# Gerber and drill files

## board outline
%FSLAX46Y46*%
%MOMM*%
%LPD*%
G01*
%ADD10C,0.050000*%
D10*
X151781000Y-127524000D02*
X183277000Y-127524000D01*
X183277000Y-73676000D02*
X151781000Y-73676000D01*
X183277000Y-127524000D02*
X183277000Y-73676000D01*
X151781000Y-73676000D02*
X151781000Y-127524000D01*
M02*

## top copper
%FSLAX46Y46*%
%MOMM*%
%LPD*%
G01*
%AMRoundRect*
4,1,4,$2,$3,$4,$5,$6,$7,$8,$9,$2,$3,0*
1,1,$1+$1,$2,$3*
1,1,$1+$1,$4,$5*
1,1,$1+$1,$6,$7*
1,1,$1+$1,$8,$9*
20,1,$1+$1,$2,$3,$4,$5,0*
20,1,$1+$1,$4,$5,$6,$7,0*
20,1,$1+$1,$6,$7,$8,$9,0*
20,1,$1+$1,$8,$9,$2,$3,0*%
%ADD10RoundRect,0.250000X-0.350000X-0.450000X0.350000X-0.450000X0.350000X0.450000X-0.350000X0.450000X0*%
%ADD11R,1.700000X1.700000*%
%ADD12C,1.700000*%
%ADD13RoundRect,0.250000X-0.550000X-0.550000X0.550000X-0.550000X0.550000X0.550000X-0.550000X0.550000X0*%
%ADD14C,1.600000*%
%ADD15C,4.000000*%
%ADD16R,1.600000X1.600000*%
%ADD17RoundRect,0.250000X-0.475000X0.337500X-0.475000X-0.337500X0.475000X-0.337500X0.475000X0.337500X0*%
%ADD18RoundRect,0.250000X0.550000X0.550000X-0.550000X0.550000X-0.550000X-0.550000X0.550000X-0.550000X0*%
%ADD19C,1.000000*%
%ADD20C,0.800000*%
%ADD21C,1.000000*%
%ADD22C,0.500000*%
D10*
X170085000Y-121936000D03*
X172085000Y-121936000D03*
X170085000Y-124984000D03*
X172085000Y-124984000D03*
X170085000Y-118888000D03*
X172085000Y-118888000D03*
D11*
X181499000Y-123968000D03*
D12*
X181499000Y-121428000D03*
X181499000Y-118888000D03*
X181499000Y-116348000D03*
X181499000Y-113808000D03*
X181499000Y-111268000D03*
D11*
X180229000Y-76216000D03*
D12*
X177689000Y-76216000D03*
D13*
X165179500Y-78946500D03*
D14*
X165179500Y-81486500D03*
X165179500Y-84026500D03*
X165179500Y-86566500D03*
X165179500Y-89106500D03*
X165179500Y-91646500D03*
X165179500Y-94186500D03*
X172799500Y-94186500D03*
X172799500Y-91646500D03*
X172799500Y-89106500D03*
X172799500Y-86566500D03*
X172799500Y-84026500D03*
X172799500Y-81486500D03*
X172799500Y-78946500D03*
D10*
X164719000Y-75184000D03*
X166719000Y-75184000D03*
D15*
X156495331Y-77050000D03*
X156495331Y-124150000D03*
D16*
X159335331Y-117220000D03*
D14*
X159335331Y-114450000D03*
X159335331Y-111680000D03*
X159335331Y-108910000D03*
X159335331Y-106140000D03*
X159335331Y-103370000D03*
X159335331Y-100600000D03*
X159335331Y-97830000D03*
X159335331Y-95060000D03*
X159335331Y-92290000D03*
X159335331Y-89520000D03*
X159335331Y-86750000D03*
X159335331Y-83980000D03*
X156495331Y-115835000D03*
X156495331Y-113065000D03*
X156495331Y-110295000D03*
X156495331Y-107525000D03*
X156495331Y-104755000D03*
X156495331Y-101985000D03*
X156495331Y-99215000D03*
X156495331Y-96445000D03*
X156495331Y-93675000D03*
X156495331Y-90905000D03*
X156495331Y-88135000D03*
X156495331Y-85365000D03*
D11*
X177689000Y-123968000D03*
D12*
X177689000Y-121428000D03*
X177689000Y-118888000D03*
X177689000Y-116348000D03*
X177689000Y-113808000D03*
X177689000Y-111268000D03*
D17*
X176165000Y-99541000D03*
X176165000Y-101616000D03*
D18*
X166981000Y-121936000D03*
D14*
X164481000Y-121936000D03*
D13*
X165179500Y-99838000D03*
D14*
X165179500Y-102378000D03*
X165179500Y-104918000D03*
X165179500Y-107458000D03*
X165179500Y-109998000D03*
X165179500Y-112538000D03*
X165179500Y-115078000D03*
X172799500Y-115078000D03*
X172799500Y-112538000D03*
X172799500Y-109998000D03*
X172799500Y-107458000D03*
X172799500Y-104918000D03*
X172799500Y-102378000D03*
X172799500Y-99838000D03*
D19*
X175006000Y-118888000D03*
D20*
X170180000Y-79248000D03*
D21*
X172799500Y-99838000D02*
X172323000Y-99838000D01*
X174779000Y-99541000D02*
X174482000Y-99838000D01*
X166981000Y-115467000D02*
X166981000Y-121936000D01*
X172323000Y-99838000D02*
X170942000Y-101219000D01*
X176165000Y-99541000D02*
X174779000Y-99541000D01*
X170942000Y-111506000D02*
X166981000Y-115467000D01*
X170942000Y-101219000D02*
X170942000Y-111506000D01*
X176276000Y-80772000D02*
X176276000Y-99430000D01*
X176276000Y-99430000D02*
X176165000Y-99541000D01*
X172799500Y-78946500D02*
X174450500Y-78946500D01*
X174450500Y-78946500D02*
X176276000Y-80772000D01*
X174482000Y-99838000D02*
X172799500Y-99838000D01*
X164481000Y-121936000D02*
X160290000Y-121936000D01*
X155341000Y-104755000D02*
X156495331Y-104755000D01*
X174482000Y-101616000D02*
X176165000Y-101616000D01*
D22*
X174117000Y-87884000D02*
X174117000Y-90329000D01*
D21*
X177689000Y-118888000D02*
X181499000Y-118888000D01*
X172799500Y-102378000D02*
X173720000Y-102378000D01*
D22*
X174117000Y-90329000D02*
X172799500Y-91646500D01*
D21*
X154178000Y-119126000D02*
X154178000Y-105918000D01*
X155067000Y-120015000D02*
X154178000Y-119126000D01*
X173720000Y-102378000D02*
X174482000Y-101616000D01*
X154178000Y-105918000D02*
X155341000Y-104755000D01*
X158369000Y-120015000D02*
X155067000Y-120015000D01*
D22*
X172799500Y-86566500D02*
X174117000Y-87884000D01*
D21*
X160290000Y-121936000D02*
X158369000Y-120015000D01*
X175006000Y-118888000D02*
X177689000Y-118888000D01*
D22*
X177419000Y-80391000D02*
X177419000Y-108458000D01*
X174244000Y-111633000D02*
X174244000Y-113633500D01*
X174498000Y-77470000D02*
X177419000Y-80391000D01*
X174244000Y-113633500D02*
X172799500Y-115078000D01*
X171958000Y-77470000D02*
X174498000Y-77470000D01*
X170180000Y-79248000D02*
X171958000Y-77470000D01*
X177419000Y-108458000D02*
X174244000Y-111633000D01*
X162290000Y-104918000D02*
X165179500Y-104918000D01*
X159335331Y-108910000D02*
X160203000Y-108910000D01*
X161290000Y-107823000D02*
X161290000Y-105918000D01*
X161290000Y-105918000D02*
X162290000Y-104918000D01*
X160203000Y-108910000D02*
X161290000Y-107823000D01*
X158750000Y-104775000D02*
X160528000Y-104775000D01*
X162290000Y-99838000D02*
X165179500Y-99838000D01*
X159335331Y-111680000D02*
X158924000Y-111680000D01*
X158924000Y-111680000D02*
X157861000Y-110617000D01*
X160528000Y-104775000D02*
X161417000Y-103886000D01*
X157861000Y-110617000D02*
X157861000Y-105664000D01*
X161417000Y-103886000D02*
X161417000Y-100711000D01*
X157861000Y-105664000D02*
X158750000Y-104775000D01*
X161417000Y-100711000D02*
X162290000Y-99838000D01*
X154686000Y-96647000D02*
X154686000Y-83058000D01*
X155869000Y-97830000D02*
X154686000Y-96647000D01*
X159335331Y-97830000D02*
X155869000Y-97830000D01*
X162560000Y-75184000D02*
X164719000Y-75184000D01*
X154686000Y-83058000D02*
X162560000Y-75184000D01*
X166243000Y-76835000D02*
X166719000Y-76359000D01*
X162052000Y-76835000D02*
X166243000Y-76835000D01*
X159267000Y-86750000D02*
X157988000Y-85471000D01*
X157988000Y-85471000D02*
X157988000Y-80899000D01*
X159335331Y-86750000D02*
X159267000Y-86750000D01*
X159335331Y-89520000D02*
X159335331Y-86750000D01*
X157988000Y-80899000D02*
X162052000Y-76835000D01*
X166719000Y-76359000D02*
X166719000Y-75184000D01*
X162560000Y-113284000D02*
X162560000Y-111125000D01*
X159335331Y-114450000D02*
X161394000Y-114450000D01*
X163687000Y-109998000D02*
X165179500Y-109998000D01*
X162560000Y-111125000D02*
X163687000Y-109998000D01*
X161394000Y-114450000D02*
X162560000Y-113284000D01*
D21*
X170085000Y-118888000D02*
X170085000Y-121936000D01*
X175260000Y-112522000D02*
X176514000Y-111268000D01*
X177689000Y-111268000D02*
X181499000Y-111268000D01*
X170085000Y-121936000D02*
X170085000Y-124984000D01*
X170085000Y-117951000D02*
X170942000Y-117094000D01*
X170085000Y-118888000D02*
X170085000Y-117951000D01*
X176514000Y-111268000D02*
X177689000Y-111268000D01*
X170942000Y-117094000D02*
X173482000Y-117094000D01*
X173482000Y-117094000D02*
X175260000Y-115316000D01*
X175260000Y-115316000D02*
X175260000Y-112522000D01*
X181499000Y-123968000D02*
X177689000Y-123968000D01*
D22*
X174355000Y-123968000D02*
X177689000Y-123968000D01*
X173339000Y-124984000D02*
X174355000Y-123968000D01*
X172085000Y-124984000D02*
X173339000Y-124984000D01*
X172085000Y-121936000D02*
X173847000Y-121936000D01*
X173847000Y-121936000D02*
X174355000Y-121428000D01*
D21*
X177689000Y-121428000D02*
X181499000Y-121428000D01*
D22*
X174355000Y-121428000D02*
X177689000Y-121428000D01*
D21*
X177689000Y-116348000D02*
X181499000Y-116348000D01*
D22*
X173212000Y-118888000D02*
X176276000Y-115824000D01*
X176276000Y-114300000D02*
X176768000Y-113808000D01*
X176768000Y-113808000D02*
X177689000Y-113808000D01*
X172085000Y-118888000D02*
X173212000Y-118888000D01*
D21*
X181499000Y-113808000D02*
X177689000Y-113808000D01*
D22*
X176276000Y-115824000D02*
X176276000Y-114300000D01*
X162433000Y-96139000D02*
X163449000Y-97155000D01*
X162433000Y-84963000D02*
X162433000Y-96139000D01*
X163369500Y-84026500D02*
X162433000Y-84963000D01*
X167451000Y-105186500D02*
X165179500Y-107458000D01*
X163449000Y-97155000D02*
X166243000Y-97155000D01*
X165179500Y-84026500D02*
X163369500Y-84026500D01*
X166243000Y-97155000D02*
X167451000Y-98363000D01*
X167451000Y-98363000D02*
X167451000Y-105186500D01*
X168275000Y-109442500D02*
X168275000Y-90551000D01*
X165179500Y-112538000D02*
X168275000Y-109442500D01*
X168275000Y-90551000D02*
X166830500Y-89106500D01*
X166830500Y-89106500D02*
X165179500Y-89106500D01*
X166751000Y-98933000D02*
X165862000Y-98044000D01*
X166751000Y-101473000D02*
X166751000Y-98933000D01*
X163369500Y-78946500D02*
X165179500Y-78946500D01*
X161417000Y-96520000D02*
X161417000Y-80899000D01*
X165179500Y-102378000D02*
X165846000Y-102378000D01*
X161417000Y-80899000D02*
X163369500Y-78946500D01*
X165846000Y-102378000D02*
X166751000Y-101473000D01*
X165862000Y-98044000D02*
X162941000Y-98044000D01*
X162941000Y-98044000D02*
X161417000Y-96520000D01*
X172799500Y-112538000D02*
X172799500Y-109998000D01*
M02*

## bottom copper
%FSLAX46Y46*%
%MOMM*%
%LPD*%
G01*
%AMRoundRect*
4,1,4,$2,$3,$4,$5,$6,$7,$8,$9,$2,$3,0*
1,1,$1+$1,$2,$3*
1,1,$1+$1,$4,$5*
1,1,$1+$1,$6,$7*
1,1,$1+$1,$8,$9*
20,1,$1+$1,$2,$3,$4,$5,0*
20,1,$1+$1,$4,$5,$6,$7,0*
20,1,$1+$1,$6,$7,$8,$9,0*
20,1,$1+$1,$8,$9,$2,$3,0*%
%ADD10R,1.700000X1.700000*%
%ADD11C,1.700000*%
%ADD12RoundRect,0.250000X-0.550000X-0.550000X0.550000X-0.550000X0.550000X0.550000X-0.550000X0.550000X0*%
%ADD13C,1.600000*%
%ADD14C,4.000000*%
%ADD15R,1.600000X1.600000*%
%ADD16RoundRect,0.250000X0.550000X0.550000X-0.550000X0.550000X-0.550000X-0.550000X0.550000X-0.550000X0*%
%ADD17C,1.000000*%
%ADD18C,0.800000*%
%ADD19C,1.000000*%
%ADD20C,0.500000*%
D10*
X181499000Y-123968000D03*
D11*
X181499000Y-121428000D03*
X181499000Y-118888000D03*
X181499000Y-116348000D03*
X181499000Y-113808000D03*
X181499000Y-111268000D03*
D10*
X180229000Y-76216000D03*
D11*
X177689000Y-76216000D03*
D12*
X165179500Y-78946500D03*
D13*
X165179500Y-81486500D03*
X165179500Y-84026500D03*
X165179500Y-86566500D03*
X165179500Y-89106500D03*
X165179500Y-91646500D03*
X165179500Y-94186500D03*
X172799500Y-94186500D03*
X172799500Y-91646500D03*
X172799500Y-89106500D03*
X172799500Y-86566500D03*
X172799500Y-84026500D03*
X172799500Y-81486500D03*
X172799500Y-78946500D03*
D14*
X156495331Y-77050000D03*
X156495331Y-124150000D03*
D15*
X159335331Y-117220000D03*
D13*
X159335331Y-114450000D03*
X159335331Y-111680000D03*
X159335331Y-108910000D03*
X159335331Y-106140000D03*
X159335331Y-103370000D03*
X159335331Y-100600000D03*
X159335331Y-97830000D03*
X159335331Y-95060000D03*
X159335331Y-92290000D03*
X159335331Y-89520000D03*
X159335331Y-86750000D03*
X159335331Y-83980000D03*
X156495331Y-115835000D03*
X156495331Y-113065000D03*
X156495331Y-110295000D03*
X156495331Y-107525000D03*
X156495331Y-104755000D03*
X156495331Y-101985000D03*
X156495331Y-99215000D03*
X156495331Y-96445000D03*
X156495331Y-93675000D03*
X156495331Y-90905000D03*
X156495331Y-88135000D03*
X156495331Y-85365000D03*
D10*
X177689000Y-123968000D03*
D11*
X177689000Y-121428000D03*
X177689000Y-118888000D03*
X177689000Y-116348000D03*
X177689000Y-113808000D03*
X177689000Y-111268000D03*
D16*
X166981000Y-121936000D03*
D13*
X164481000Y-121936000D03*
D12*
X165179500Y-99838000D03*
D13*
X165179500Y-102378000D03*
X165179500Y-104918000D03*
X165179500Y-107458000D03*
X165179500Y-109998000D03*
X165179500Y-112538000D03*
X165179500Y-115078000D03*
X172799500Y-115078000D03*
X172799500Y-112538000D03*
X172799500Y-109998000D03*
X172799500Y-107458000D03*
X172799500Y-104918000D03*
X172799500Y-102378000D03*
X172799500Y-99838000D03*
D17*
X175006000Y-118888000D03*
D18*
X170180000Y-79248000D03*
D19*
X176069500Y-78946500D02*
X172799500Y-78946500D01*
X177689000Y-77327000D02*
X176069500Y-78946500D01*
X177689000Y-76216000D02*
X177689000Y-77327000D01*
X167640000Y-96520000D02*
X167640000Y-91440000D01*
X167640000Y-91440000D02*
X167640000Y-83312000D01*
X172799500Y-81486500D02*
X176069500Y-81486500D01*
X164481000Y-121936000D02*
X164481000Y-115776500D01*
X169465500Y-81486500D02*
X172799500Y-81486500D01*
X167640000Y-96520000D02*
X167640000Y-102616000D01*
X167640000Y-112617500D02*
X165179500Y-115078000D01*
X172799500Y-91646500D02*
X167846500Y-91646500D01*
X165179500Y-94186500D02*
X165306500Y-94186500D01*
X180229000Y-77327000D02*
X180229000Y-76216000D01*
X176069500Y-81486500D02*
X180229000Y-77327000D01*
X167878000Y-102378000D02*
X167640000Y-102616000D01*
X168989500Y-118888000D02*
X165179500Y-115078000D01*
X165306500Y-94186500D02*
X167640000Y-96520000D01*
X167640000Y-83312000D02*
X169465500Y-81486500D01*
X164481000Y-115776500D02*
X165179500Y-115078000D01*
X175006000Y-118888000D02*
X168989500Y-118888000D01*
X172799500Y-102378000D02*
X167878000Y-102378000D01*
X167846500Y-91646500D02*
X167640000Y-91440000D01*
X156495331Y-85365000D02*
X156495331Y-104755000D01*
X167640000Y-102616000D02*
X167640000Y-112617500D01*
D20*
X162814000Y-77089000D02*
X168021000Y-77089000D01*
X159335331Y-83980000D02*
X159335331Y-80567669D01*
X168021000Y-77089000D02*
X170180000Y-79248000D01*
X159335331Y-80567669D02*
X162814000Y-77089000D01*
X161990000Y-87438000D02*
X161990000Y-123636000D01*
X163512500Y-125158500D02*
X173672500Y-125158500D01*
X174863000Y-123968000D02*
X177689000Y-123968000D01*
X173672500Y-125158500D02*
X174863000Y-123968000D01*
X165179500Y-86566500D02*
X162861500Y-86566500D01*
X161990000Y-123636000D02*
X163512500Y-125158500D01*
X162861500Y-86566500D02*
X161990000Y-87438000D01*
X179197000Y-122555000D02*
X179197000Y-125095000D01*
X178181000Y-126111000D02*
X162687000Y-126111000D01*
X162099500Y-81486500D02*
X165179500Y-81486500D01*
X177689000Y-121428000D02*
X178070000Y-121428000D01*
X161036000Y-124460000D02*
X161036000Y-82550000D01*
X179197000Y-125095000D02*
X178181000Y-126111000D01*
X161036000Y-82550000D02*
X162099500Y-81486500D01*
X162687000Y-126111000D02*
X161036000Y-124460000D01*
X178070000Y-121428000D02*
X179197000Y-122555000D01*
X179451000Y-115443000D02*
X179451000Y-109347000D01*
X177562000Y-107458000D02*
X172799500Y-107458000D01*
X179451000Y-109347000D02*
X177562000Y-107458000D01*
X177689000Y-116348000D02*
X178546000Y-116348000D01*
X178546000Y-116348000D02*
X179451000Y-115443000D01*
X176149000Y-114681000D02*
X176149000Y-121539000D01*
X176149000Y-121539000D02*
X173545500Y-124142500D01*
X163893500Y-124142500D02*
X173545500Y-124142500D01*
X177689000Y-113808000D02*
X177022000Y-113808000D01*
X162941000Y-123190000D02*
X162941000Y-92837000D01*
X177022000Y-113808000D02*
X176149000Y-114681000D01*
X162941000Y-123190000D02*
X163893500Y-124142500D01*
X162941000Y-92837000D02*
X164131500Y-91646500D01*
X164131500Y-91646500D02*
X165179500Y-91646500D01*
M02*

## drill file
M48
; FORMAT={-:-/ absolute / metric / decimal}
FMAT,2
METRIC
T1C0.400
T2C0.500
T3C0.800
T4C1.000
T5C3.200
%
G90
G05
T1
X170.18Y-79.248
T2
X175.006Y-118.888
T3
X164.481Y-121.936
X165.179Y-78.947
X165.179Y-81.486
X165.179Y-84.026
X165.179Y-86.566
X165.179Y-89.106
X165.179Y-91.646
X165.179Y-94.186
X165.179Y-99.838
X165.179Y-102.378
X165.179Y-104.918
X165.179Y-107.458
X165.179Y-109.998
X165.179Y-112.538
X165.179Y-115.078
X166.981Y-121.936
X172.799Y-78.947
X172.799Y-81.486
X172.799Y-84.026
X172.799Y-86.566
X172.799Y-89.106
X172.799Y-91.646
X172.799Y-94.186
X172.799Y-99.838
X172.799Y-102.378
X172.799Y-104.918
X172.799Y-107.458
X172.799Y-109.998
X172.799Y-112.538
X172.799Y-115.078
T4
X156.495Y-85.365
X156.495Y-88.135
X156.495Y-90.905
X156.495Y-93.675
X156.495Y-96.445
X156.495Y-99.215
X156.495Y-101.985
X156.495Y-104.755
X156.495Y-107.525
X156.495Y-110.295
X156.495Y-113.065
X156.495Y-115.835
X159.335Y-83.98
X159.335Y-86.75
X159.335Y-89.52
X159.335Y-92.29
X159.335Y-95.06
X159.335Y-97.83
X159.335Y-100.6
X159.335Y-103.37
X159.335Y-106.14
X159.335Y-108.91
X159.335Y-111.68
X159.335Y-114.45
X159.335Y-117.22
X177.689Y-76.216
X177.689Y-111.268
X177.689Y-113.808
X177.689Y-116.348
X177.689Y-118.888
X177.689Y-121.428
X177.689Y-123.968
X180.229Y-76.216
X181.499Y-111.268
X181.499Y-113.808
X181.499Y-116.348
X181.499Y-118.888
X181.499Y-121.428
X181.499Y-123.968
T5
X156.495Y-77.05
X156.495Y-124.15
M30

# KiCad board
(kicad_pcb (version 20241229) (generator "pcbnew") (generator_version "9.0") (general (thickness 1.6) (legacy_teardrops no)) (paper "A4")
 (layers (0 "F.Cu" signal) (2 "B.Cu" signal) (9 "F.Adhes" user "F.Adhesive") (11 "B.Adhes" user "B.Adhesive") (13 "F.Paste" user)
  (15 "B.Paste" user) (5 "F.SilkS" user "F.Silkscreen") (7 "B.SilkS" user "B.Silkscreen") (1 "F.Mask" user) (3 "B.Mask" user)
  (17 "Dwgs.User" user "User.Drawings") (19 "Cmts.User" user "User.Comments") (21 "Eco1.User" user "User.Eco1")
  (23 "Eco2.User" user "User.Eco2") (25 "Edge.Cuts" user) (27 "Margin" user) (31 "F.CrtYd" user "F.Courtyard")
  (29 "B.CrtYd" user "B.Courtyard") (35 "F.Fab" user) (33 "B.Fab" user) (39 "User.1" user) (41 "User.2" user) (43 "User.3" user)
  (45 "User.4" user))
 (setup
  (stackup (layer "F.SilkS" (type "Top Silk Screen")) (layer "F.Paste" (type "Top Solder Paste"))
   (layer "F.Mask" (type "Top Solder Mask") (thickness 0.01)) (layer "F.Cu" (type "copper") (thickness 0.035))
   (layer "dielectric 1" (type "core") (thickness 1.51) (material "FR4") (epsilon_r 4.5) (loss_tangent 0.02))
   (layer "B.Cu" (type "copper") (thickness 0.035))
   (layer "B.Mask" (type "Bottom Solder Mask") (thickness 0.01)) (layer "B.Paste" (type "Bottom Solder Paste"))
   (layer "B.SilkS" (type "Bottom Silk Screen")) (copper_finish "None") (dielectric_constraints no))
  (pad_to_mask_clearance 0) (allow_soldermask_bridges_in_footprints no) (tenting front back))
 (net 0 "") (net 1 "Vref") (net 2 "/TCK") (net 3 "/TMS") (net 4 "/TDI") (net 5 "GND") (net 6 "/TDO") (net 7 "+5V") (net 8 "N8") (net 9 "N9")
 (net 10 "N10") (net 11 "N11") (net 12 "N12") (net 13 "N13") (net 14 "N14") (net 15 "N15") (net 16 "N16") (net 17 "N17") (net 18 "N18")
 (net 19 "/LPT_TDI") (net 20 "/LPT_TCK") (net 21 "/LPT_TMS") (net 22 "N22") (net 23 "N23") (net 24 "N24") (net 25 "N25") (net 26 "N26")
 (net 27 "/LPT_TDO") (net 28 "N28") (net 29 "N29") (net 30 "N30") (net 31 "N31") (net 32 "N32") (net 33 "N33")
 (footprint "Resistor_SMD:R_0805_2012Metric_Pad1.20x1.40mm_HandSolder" (layer "F.Cu") (at 171.085 121.936)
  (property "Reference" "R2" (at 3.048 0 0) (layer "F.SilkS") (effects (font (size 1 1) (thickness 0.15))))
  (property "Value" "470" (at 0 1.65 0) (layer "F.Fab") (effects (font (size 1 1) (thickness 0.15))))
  (pad "1" smd roundrect (at -1 0) (size 1.2 1.4) (layers "F.Cu" "F.Mask" "F.Paste") (roundrect_rratio 0.208333) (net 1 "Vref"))
  (pad "2" smd roundrect (at 1 0) (size 1.2 1.4) (layers "F.Cu" "F.Mask" "F.Paste") (roundrect_rratio 0.208333) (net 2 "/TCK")))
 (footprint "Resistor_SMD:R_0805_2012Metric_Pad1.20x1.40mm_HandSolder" (layer "F.Cu") (at 171.085 124.984)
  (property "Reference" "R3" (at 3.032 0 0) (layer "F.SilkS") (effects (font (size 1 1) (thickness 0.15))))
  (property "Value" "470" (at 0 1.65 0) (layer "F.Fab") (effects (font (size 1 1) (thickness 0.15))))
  (pad "1" smd roundrect (at -1 0) (size 1.2 1.4) (layers "F.Cu" "F.Mask" "F.Paste") (roundrect_rratio 0.208333) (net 1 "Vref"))
  (pad "2" smd roundrect (at 1 0) (size 1.2 1.4) (layers "F.Cu" "F.Mask" "F.Paste") (roundrect_rratio 0.208333) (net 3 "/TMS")))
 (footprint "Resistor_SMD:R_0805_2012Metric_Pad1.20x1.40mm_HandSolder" (layer "F.Cu") (at 171.085 118.888)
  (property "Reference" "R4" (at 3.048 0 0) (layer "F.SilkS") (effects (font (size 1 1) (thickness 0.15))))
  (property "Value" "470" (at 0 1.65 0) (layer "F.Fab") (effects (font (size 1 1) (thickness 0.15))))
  (pad "1" smd roundrect (at -1 0) (size 1.2 1.4) (layers "F.Cu" "F.Mask" "F.Paste") (roundrect_rratio 0.208333) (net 1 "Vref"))
  (pad "2" smd roundrect (at 1 0) (size 1.2 1.4) (layers "F.Cu" "F.Mask" "F.Paste") (roundrect_rratio 0.208333) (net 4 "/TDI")))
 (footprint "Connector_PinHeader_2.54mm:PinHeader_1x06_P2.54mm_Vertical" (layer "F.Cu") (at 181.499 123.968 180)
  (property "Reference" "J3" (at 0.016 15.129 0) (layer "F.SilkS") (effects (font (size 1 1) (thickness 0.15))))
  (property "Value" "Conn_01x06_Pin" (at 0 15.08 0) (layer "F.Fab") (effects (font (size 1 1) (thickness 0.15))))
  (pad "1" thru_hole rect (at 0 0 180) (size 1.7 1.7) (drill 1) (layers "*.Cu" "*.Mask") (remove_unused_layers no) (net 3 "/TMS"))
  (pad "2" thru_hole circle (at 0 2.54 180) (size 1.7 1.7) (drill 1) (layers "*.Cu" "*.Mask") (remove_unused_layers no) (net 2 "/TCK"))
  (pad "3" thru_hole circle (at 0 5.08 180) (size 1.7 1.7) (drill 1) (layers "*.Cu" "*.Mask") (remove_unused_layers no) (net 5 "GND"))
  (pad "4" thru_hole circle (at 0 7.62 180) (size 1.7 1.7) (drill 1) (layers "*.Cu" "*.Mask") (remove_unused_layers no) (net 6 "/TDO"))
  (pad "5" thru_hole circle (at 0 10.16 180) (size 1.7 1.7) (drill 1) (layers "*.Cu" "*.Mask") (remove_unused_layers no) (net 4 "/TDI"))
  (pad "6" thru_hole circle (at 0 12.7 180) (size 1.7 1.7) (drill 1) (layers "*.Cu" "*.Mask") (remove_unused_layers no) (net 1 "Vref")))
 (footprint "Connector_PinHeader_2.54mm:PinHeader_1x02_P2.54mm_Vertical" (layer "F.Cu") (at 180.229 76.216 -90)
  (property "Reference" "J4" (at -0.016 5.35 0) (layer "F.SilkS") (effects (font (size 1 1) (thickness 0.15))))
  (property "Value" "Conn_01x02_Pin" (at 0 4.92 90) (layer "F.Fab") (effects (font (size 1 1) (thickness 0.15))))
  (pad "1" thru_hole rect (at 0 0 270) (size 1.7 1.7) (drill 1) (layers "*.Cu" "*.Mask") (remove_unused_layers no) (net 5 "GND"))
  (pad "2" thru_hole circle (at 0 2.54 270) (size 1.7 1.7) (drill 1) (layers "*.Cu" "*.Mask") (remove_unused_layers no) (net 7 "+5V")))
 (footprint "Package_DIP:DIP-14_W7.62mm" (layer "F.Cu") (at 165.1795 78.9465)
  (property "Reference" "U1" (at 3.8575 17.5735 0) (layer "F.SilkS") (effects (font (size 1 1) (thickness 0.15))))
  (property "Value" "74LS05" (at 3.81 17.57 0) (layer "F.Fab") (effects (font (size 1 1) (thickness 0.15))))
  (pad "1" thru_hole roundrect (at 0 0) (size 1.6 1.6) (drill 0.8) (layers "*.Cu" "*.Mask") (remove_unused_layers no)
   (roundrect_rratio 0.15625) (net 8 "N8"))
  (pad "2" thru_hole circle (at 0 2.54) (size 1.6 1.6) (drill 0.8) (layers "*.Cu" "*.Mask") (remove_unused_layers no) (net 2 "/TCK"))
  (pad "3" thru_hole circle (at 0 5.08) (size 1.6 1.6) (drill 0.8) (layers "*.Cu" "*.Mask") (remove_unused_layers no) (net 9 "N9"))
  (pad "4" thru_hole circle (at 0 7.62) (size 1.6 1.6) (drill 0.8) (layers "*.Cu" "*.Mask") (remove_unused_layers no) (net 3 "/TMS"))
  (pad "5" thru_hole circle (at 0 10.16) (size 1.6 1.6) (drill 0.8) (layers "*.Cu" "*.Mask") (remove_unused_layers no) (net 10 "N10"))
  (pad "6" thru_hole circle (at 0 12.7) (size 1.6 1.6) (drill 0.8) (layers "*.Cu" "*.Mask") (remove_unused_layers no) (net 4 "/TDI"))
  (pad "7" thru_hole circle (at 0 15.24) (size 1.6 1.6) (drill 0.8) (layers "*.Cu" "*.Mask") (remove_unused_layers no) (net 5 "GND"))
  (pad "8" thru_hole circle (at 7.62 15.24) (size 1.6 1.6) (drill 0.8) (layers "*.Cu" "*.Mask") (remove_unused_layers no) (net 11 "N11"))
  (pad "9" thru_hole circle (at 7.62 12.7) (size 1.6 1.6) (drill 0.8) (layers "*.Cu" "*.Mask") (remove_unused_layers no) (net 5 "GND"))
  (pad "10" thru_hole circle (at 7.62 10.16) (size 1.6 1.6) (drill 0.8) (layers "*.Cu" "*.Mask") (remove_unused_layers no) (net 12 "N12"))
  (pad "11" thru_hole circle (at 7.62 7.62) (size 1.6 1.6) (drill 0.8) (layers "*.Cu" "*.Mask") (remove_unused_layers no) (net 5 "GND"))
  (pad "12" thru_hole circle (at 7.62 5.08) (size 1.6 1.6) (drill 0.8) (layers "*.Cu" "*.Mask") (remove_unused_layers no) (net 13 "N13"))
  (pad "13" thru_hole circle (at 7.62 2.54) (size 1.6 1.6) (drill 0.8) (layers "*.Cu" "*.Mask") (remove_unused_layers no) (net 5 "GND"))
  (pad "14" thru_hole circle (at 7.62 0) (size 1.6 1.6) (drill 0.8) (layers "*.Cu" "*.Mask") (remove_unused_layers no) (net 7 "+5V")))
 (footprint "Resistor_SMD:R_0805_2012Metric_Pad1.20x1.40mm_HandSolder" (layer "F.Cu") (at 165.719 75.184)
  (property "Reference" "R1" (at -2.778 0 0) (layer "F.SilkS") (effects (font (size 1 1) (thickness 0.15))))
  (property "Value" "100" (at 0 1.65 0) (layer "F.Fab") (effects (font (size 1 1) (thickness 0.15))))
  (pad "1" smd roundrect (at -1 0) (size 1.2 1.4) (layers "F.Cu" "F.Mask" "F.Paste") (roundrect_rratio 0.208333) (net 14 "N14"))
  (pad "2" smd roundrect (at 1 0) (size 1.2 1.4) (layers "F.Cu" "F.Mask" "F.Paste") (roundrect_rratio 0.208333) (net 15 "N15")))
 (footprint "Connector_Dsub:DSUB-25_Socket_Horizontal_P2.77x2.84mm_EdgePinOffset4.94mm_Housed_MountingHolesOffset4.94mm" (layer "F.Cu")
  (at 159.335331 117.22 -90)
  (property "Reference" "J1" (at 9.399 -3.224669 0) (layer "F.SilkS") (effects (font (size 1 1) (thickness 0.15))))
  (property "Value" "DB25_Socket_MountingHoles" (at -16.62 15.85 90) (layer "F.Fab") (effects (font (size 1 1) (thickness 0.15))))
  (pad "0" thru_hole circle (at -40.17 2.84 270) (size 4 4) (drill 3.2) (layers "*.Cu" "*.Mask") (remove_unused_layers no) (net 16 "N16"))
  (pad "0" thru_hole circle (at 6.93 2.84 270) (size 4 4) (drill 3.2) (layers "*.Cu" "*.Mask") (remove_unused_layers no) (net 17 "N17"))
  (pad "1" thru_hole rect (at 0 0 270) (size 1.6 1.6) (drill 1) (layers "*.Cu" "*.Mask") (remove_unused_layers no) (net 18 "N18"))
  (pad "2" thru_hole circle (at -2.77 0 270) (size 1.6 1.6) (drill 1) (layers "*.Cu" "*.Mask") (remove_unused_layers no) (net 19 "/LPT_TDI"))
  (pad "3" thru_hole circle (at -5.54 0 270) (size 1.6 1.6) (drill 1) (layers "*.Cu" "*.Mask") (remove_unused_layers no) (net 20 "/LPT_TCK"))
  (pad "4" thru_hole circle (at -8.31 0 270) (size 1.6 1.6) (drill 1) (layers "*.Cu" "*.Mask") (remove_unused_layers no) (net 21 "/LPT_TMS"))
  (pad "5" thru_hole circle (at -11.08 0 270) (size 1.6 1.6) (drill 1) (layers "*.Cu" "*.Mask") (remove_unused_layers no) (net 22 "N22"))
  (pad "6" thru_hole circle (at -13.85 0 270) (size 1.6 1.6) (drill 1) (layers "*.Cu" "*.Mask") (remove_unused_layers no) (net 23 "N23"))
  (pad "7" thru_hole circle (at -16.62 0 270) (size 1.6 1.6) (drill 1) (layers "*.Cu" "*.Mask") (remove_unused_layers no) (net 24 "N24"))
  (pad "8" thru_hole circle (at -19.39 0 270) (size 1.6 1.6) (drill 1) (layers "*.Cu" "*.Mask") (remove_unused_layers no) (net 14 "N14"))
  (pad "9" thru_hole circle (at -22.16 0 270) (size 1.6 1.6) (drill 1) (layers "*.Cu" "*.Mask") (remove_unused_layers no) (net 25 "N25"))
  (pad "10" thru_hole circle (at -24.93 0 270) (size 1.6 1.6) (drill 1) (layers "*.Cu" "*.Mask") (remove_unused_layers no) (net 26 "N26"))
  (pad "11" thru_hole circle (at -27.7 0 270) (size 1.6 1.6) (drill 1) (layers "*.Cu" "*.Mask") (remove_unused_layers no) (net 15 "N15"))
  (pad "12" thru_hole circle (at -30.47 0 270) (size 1.6 1.6) (drill 1) (layers "*.Cu" "*.Mask") (remove_unused_layers no) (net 15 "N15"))
  (pad "13" thru_hole circle (at -33.24 0 270) (size 1.6 1.6) (drill 1) (layers "*.Cu" "*.Mask") (remove_unused_layers no)
   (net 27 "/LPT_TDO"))
  (pad "14" thru_hole circle (at -1.385 2.84 270) (size 1.6 1.6) (drill 1) (layers "*.Cu" "*.Mask") (remove_unused_layers no) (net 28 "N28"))
  (pad "15" thru_hole circle (at -4.155 2.84 270) (size 1.6 1.6) (drill 1) (layers "*.Cu" "*.Mask") (remove_unused_layers no) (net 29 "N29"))
  (pad "16" thru_hole circle (at -6.925 2.84 270) (size 1.6 1.6) (drill 1) (layers "*.Cu" "*.Mask") (remove_unused_layers no) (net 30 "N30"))
  (pad "17" thru_hole circle (at -9.695 2.84 270) (size 1.6 1.6) (drill 1) (layers "*.Cu" "*.Mask") (remove_unused_layers no) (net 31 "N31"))
  (pad "18" thru_hole circle (at -12.465 2.84 270) (size 1.6 1.6) (drill 1) (layers "*.Cu" "*.Mask") (remove_unused_layers no) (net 5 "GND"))
  (pad "19" thru_hole circle (at -15.235 2.84 270) (size 1.6 1.6) (drill 1) (layers "*.Cu" "*.Mask") (remove_unused_layers no) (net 5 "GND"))
  (pad "20" thru_hole circle (at -18.005 2.84 270) (size 1.6 1.6) (drill 1) (layers "*.Cu" "*.Mask") (remove_unused_layers no) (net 5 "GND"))
  (pad "21" thru_hole circle (at -20.775 2.84 270) (size 1.6 1.6) (drill 1) (layers "*.Cu" "*.Mask") (remove_unused_layers no) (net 5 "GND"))
  (pad "22" thru_hole circle (at -23.545 2.84 270) (size 1.6 1.6) (drill 1) (layers "*.Cu" "*.Mask") (remove_unused_layers no) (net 5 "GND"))
  (pad "23" thru_hole circle (at -26.315 2.84 270) (size 1.6 1.6) (drill 1) (layers "*.Cu" "*.Mask") (remove_unused_layers no) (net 5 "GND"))
  (pad "24" thru_hole circle (at -29.085 2.84 270) (size 1.6 1.6) (drill 1) (layers "*.Cu" "*.Mask") (remove_unused_layers no) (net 5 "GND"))
  (pad "25" thru_hole circle (at -31.855 2.84 270) (size 1.6 1.6) (drill 1) (layers "*.Cu" "*.Mask") (remove_unused_layers no) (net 5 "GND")))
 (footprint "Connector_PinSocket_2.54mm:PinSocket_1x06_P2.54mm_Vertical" (layer "F.Cu") (at 177.689 123.968 180)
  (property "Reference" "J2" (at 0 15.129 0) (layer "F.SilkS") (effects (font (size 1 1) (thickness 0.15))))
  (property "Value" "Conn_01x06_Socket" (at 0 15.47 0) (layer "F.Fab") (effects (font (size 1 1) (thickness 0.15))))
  (pad "1" thru_hole rect (at 0 0 180) (size 1.7 1.7) (drill 1) (layers "*.Cu" "*.Mask") (remove_unused_layers no) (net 3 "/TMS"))
  (pad "2" thru_hole circle (at 0 2.54 180) (size 1.7 1.7) (drill 1) (layers "*.Cu" "*.Mask") (remove_unused_layers no) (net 2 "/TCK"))
  (pad "3" thru_hole circle (at 0 5.08 180) (size 1.7 1.7) (drill 1) (layers "*.Cu" "*.Mask") (remove_unused_layers no) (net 5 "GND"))
  (pad "4" thru_hole circle (at 0 7.62 180) (size 1.7 1.7) (drill 1) (layers "*.Cu" "*.Mask") (remove_unused_layers no) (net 6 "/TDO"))
  (pad "5" thru_hole circle (at 0 10.16 180) (size 1.7 1.7) (drill 1) (layers "*.Cu" "*.Mask") (remove_unused_layers no) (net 4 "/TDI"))
  (pad "6" thru_hole circle (at 0 12.7 180) (size 1.7 1.7) (drill 1) (layers "*.Cu" "*.Mask") (remove_unused_layers no) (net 1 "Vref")))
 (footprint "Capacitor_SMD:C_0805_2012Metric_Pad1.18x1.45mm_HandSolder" (layer "F.Cu") (at 176.165 100.5785 -90)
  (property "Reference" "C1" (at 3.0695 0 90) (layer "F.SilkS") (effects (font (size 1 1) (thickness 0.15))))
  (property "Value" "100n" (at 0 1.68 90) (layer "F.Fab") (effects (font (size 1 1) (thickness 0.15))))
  (pad "1" smd roundrect (at -1.0375 0 270) (size 1.175 1.45) (layers "F.Cu" "F.Mask" "F.Paste") (roundrect_rratio 0.212766) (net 7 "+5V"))
  (pad "2" smd roundrect (at 1.0375 0 270) (size 1.175 1.45) (layers "F.Cu" "F.Mask" "F.Paste") (roundrect_rratio 0.212766) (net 5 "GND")))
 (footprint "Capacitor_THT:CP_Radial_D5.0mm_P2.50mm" (layer "F.Cu") (at 166.981 121.936 180)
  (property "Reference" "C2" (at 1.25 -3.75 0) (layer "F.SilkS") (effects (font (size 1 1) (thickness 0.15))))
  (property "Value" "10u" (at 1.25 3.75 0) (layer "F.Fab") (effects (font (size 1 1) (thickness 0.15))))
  (pad "1" thru_hole roundrect (at 0 0 180) (size 1.6 1.6) (drill 0.8) (layers "*.Cu" "*.Mask") (remove_unused_layers no)
   (roundrect_rratio 0.15625) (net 7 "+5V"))
  (pad "2" thru_hole circle (at 2.5 0 180) (size 1.6 1.6) (drill 0.8) (layers "*.Cu" "*.Mask") (remove_unused_layers no) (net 5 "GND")))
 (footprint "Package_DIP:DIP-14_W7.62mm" (layer "F.Cu") (at 165.1795 99.838)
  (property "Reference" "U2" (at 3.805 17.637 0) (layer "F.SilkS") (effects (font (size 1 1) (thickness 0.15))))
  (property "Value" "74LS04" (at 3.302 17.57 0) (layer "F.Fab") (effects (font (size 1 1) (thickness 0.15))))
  (pad "1" thru_hole roundrect (at 0 0) (size 1.6 1.6) (drill 0.8) (layers "*.Cu" "*.Mask") (remove_unused_layers no)
   (roundrect_rratio 0.15625) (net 20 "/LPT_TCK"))
  (pad "2" thru_hole circle (at 0 2.54) (size 1.6 1.6) (drill 0.8) (layers "*.Cu" "*.Mask") (remove_unused_layers no) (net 8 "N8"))
  (pad "3" thru_hole circle (at 0 5.08) (size 1.6 1.6) (drill 0.8) (layers "*.Cu" "*.Mask") (remove_unused_layers no) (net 21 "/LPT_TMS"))
  (pad "4" thru_hole circle (at 0 7.62) (size 1.6 1.6) (drill 0.8) (layers "*.Cu" "*.Mask") (remove_unused_layers no) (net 9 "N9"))
  (pad "5" thru_hole circle (at 0 10.16) (size 1.6 1.6) (drill 0.8) (layers "*.Cu" "*.Mask") (remove_unused_layers no) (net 19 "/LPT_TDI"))
  (pad "6" thru_hole circle (at 0 12.7) (size 1.6 1.6) (drill 0.8) (layers "*.Cu" "*.Mask") (remove_unused_layers no) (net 10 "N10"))
  (pad "7" thru_hole circle (at 0 15.24) (size 1.6 1.6) (drill 0.8) (layers "*.Cu" "*.Mask") (remove_unused_layers no) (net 5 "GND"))
  (pad "8" thru_hole circle (at 7.62 15.24) (size 1.6 1.6) (drill 0.8) (layers "*.Cu" "*.Mask") (remove_unused_layers no)
   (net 27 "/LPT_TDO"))
  (pad "9" thru_hole circle (at 7.62 12.7) (size 1.6 1.6) (drill 0.8) (layers "*.Cu" "*.Mask") (remove_unused_layers no) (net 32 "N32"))
  (pad "10" thru_hole circle (at 7.62 10.16) (size 1.6 1.6) (drill 0.8) (layers "*.Cu" "*.Mask") (remove_unused_layers no) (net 32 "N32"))
  (pad "11" thru_hole circle (at 7.62 7.62) (size 1.6 1.6) (drill 0.8) (layers "*.Cu" "*.Mask") (remove_unused_layers no) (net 6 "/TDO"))
  (pad "12" thru_hole circle (at 7.62 5.08) (size 1.6 1.6) (drill 0.8) (layers "*.Cu" "*.Mask") (remove_unused_layers no) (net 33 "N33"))
  (pad "13" thru_hole circle (at 7.62 2.54) (size 1.6 1.6) (drill 0.8) (layers "*.Cu" "*.Mask") (remove_unused_layers no) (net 5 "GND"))
  (pad "14" thru_hole circle (at 7.62 0) (size 1.6 1.6) (drill 0.8) (layers "*.Cu" "*.Mask") (remove_unused_layers no) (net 7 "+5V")))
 (gr_line (start 151.781 127.524) (end 183.277 127.524) (stroke (width 0.05) (type default)) (layer "Edge.Cuts"))
 (gr_line (start 183.277 73.676) (end 151.781 73.676) (stroke (width 0.05) (type default)) (layer "Edge.Cuts"))
 (gr_line (start 183.277 127.524) (end 183.277 73.676) (stroke (width 0.05) (type default)) (layer "Edge.Cuts"))
 (gr_line (start 151.781 73.676) (end 151.781 127.524) (stroke (width 0.05) (type default)) (layer "Edge.Cuts"))
 (segment (start 172.7995 99.838) (end 172.323 99.838) (width 1) (layer "F.Cu") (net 7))
 (segment (start 174.779 99.541) (end 174.482 99.838) (width 1) (layer "F.Cu") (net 7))
 (segment (start 166.981 115.467) (end 166.981 121.936) (width 1) (layer "F.Cu") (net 7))
 (segment (start 172.323 99.838) (end 170.942 101.219) (width 1) (layer "F.Cu") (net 7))
 (segment (start 176.165 99.541) (end 174.779 99.541) (width 1) (layer "F.Cu") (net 7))
 (segment (start 170.942 111.506) (end 166.981 115.467) (width 1) (layer "F.Cu") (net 7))
 (segment (start 170.942 101.219) (end 170.942 111.506) (width 1) (layer "F.Cu") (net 7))
 (segment (start 176.276 80.772) (end 176.276 99.43) (width 1) (layer "F.Cu") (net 7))
 (segment (start 176.276 99.43) (end 176.165 99.541) (width 1) (layer "F.Cu") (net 7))
 (segment (start 172.7995 78.9465) (end 174.4505 78.9465) (width 1) (layer "F.Cu") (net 7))
 (segment (start 174.4505 78.9465) (end 176.276 80.772) (width 1) (layer "F.Cu") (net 7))
 (segment (start 174.482 99.838) (end 172.7995 99.838) (width 1) (layer "F.Cu") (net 7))
 (segment (start 176.0695 78.9465) (end 172.7995 78.9465) (width 1) (layer "B.Cu") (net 7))
 (segment (start 177.689 77.327) (end 176.0695 78.9465) (width 1) (layer "B.Cu") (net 7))
 (segment (start 177.689 76.216) (end 177.689 77.327) (width 1) (layer "B.Cu") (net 7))
 (segment (start 164.481 121.936) (end 160.29 121.936) (width 1) (layer "F.Cu") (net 5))
 (segment (start 155.341 104.755) (end 156.495331 104.755) (width 1) (layer "F.Cu") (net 5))
 (segment (start 174.482 101.616) (end 176.165 101.616) (width 1) (layer "F.Cu") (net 5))
 (segment (start 174.117 87.884) (end 174.117 90.329) (width 0.5) (layer "F.Cu") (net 5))
 (segment (start 177.689 118.888) (end 181.499 118.888) (width 1) (layer "F.Cu") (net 5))
 (segment (start 172.7995 102.378) (end 173.72 102.378) (width 1) (layer "F.Cu") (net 5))
 (segment (start 174.117 90.329) (end 172.7995 91.6465) (width 0.5) (layer "F.Cu") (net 5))
 (segment (start 154.178 119.126) (end 154.178 105.918) (width 1) (layer "F.Cu") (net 5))
 (segment (start 155.067 120.015) (end 154.178 119.126) (width 1) (layer "F.Cu") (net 5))
 (segment (start 173.72 102.378) (end 174.482 101.616) (width 1) (layer "F.Cu") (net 5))
 (segment (start 154.178 105.918) (end 155.341 104.755) (width 1) (layer "F.Cu") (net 5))
 (segment (start 158.369 120.015) (end 155.067 120.015) (width 1) (layer "F.Cu") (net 5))
 (segment (start 172.7995 86.5665) (end 174.117 87.884) (width 0.5) (layer "F.Cu") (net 5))
 (segment (start 160.29 121.936) (end 158.369 120.015) (width 1) (layer "F.Cu") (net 5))
 (segment (start 175.006 118.888) (end 177.689 118.888) (width 1) (layer "F.Cu") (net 5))
 (via (at 175.006 118.888) (size 1) (drill 0.5) (layers "F.Cu" "B.Cu") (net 5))
 (segment (start 167.64 96.52) (end 167.64 91.44) (width 1) (layer "B.Cu") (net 5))
 (segment (start 167.64 91.44) (end 167.64 83.312) (width 1) (layer "B.Cu") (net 5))
 (segment (start 172.7995 81.4865) (end 176.0695 81.4865) (width 1) (layer "B.Cu") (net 5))
 (segment (start 164.481 121.936) (end 164.481 115.7765) (width 1) (layer "B.Cu") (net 5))
 (segment (start 169.4655 81.4865) (end 172.7995 81.4865) (width 1) (layer "B.Cu") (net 5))
 (segment (start 167.64 96.52) (end 167.64 102.616) (width 1) (layer "B.Cu") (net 5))
 (segment (start 167.64 112.6175) (end 165.1795 115.078) (width 1) (layer "B.Cu") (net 5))
 (segment (start 172.7995 91.6465) (end 167.8465 91.6465) (width 1) (layer "B.Cu") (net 5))
 (segment (start 165.1795 94.1865) (end 165.3065 94.1865) (width 1) (layer "B.Cu") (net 5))
 (segment (start 180.229 77.327) (end 180.229 76.216) (width 1) (layer "B.Cu") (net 5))
 (segment (start 176.0695 81.4865) (end 180.229 77.327) (width 1) (layer "B.Cu") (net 5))
 (segment (start 167.878 102.378) (end 167.64 102.616) (width 1) (layer "B.Cu") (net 5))
 (segment (start 168.9895 118.888) (end 165.1795 115.078) (width 1) (layer "B.Cu") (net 5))
 (segment (start 165.3065 94.1865) (end 167.64 96.52) (width 1) (layer "B.Cu") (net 5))
 (segment (start 167.64 83.312) (end 169.4655 81.4865) (width 1) (layer "B.Cu") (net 5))
 (segment (start 164.481 115.7765) (end 165.1795 115.078) (width 1) (layer "B.Cu") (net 5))
 (segment (start 175.006 118.888) (end 168.9895 118.888) (width 1) (layer "B.Cu") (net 5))
 (segment (start 172.7995 102.378) (end 167.878 102.378) (width 1) (layer "B.Cu") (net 5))
 (segment (start 167.8465 91.6465) (end 167.64 91.44) (width 1) (layer "B.Cu") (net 5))
 (segment (start 156.495331 85.365) (end 156.495331 104.755) (width 1) (layer "B.Cu") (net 5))
 (segment (start 167.64 102.616) (end 167.64 112.6175) (width 1) (layer "B.Cu") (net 5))
 (segment (start 177.419 80.391) (end 177.419 108.458) (width 0.5) (layer "F.Cu") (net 27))
 (segment (start 174.244 111.633) (end 174.244 113.6335) (width 0.5) (layer "F.Cu") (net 27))
 (segment (start 174.498 77.47) (end 177.419 80.391) (width 0.5) (layer "F.Cu") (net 27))
 (segment (start 174.244 113.6335) (end 172.7995 115.078) (width 0.5) (layer "F.Cu") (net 27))
 (segment (start 171.958 77.47) (end 174.498 77.47) (width 0.5) (layer "F.Cu") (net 27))
 (segment (start 170.18 79.248) (end 171.958 77.47) (width 0.5) (layer "F.Cu") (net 27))
 (segment (start 177.419 108.458) (end 174.244 111.633) (width 0.5) (layer "F.Cu") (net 27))
 (via (at 170.18 79.248) (size 0.8) (drill 0.4) (layers "F.Cu" "B.Cu") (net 27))
 (segment (start 162.814 77.089) (end 168.021 77.089) (width 0.5) (layer "B.Cu") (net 27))
 (segment (start 159.335331 83.98) (end 159.335331 80.567669) (width 0.5) (layer "B.Cu") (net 27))
 (segment (start 168.021 77.089) (end 170.18 79.248) (width 0.5) (layer "B.Cu") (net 27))
 (segment (start 159.335331 80.567669) (end 162.814 77.089) (width 0.5) (layer "B.Cu") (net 27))
 (segment (start 162.29 104.918) (end 165.1795 104.918) (width 0.5) (layer "F.Cu") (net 21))
 (segment (start 159.335331 108.91) (end 160.203 108.91) (width 0.5) (layer "F.Cu") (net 21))
 (segment (start 161.29 107.823) (end 161.29 105.918) (width 0.5) (layer "F.Cu") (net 21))
 (segment (start 161.29 105.918) (end 162.29 104.918) (width 0.5) (layer "F.Cu") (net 21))
 (segment (start 160.203 108.91) (end 161.29 107.823) (width 0.5) (layer "F.Cu") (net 21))
 (segment (start 158.75 104.775) (end 160.528 104.775) (width 0.5) (layer "F.Cu") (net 20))
 (segment (start 162.29 99.838) (end 165.1795 99.838) (width 0.5) (layer "F.Cu") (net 20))
 (segment (start 159.335331 111.68) (end 158.924 111.68) (width 0.5) (layer "F.Cu") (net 20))
 (segment (start 158.924 111.68) (end 157.861 110.617) (width 0.5) (layer "F.Cu") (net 20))
 (segment (start 160.528 104.775) (end 161.417 103.886) (width 0.5) (layer "F.Cu") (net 20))
 (segment (start 157.861 110.617) (end 157.861 105.664) (width 0.5) (layer "F.Cu") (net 20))
 (segment (start 161.417 103.886) (end 161.417 100.711) (width 0.5) (layer "F.Cu") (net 20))
 (segment (start 157.861 105.664) (end 158.75 104.775) (width 0.5) (layer "F.Cu") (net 20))
 (segment (start 161.417 100.711) (end 162.29 99.838) (width 0.5) (layer "F.Cu") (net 20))
 (segment (start 154.686 96.647) (end 154.686 83.058) (width 0.5) (layer "F.Cu") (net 14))
 (segment (start 155.869 97.83) (end 154.686 96.647) (width 0.5) (layer "F.Cu") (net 14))
 (segment (start 159.335331 97.83) (end 155.869 97.83) (width 0.5) (layer "F.Cu") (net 14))
 (segment (start 162.56 75.184) (end 164.719 75.184) (width 0.5) (layer "F.Cu") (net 14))
 (segment (start 154.686 83.058) (end 162.56 75.184) (width 0.5) (layer "F.Cu") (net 14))
 (segment (start 166.243 76.835) (end 166.719 76.359) (width 0.5) (layer "F.Cu") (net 15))
 (segment (start 162.052 76.835) (end 166.243 76.835) (width 0.5) (layer "F.Cu") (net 15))
 (segment (start 159.267 86.75) (end 157.988 85.471) (width 0.5) (layer "F.Cu") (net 15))
 (segment (start 157.988 85.471) (end 157.988 80.899) (width 0.5) (layer "F.Cu") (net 15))
 (segment (start 159.335331 86.75) (end 159.267 86.75) (width 0.5) (layer "F.Cu") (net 15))
 (segment (start 159.335331 89.52) (end 159.335331 86.75) (width 0.5) (layer "F.Cu") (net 15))
 (segment (start 157.988 80.899) (end 162.052 76.835) (width 0.5) (layer "F.Cu") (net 15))
 (segment (start 166.719 76.359) (end 166.719 75.184) (width 0.5) (layer "F.Cu") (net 15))
 (segment (start 162.56 113.284) (end 162.56 111.125) (width 0.5) (layer "F.Cu") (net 19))
 (segment (start 159.335331 114.45) (end 161.394 114.45) (width 0.5) (layer "F.Cu") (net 19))
 (segment (start 163.687 109.998) (end 165.1795 109.998) (width 0.5) (layer "F.Cu") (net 19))
 (segment (start 162.56 111.125) (end 163.687 109.998) (width 0.5) (layer "F.Cu") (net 19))
 (segment (start 161.394 114.45) (end 162.56 113.284) (width 0.5) (layer "F.Cu") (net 19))
 (segment (start 170.085 118.888) (end 170.085 121.936) (width 1) (layer "F.Cu") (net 1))
 (segment (start 175.26 112.522) (end 176.514 111.268) (width 1) (layer "F.Cu") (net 1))
 (segment (start 177.689 111.268) (end 181.499 111.268) (width 1) (layer "F.Cu") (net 1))
 (segment (start 170.085 121.936) (end 170.085 124.984) (width 1) (layer "F.Cu") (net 1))
 (segment (start 170.085 117.951) (end 170.942 117.094) (width 1) (layer "F.Cu") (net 1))
 (segment (start 170.085 118.888) (end 170.085 117.951) (width 1) (layer "F.Cu") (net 1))
 (segment (start 176.514 111.268) (end 177.689 111.268) (width 1) (layer "F.Cu") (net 1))
 (segment (start 170.942 117.094) (end 173.482 117.094) (width 1) (layer "F.Cu") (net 1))
 (segment (start 173.482 117.094) (end 175.26 115.316) (width 1) (layer "F.Cu") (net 1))
 (segment (start 175.26 115.316) (end 175.26 112.522) (width 1) (layer "F.Cu") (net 1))
 (segment (start 181.499 123.968) (end 177.689 123.968) (width 1) (layer "F.Cu") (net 3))
 (segment (start 174.355 123.968) (end 177.689 123.968) (width 0.5) (layer "F.Cu") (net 3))
 (segment (start 173.339 124.984) (end 174.355 123.968) (width 0.5) (layer "F.Cu") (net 3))
 (segment (start 172.085 124.984) (end 173.339 124.984) (width 0.5) (layer "F.Cu") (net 3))
 (segment (start 161.99 87.438) (end 161.99 123.636) (width 0.5) (layer "B.Cu") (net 3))
 (segment (start 163.5125 125.1585) (end 173.6725 125.1585) (width 0.5) (layer "B.Cu") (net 3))
 (segment (start 174.863 123.968) (end 177.689 123.968) (width 0.5) (layer "B.Cu") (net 3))
 (segment (start 173.6725 125.1585) (end 174.863 123.968) (width 0.5) (layer "B.Cu") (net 3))
 (segment (start 165.1795 86.5665) (end 162.8615 86.5665) (width 0.5) (layer "B.Cu") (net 3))
 (segment (start 161.99 123.636) (end 163.5125 125.1585) (width 0.5) (layer "B.Cu") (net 3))
 (segment (start 162.8615 86.5665) (end 161.99 87.438) (width 0.5) (layer "B.Cu") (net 3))
 (segment (start 172.085 121.936) (end 173.847 121.936) (width 0.5) (layer "F.Cu") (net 2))
 (segment (start 173.847 121.936) (end 174.355 121.428) (width 0.5) (layer "F.Cu") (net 2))
 (segment (start 177.689 121.428) (end 181.499 121.428) (width 1) (layer "F.Cu") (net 2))
 (segment (start 174.355 121.428) (end 177.689 121.428) (width 0.5) (layer "F.Cu") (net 2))
 (segment (start 179.197 122.555) (end 179.197 125.095) (width 0.5) (layer "B.Cu") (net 2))
 (segment (start 178.181 126.111) (end 162.687 126.111) (width 0.5) (layer "B.Cu") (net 2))
 (segment (start 162.0995 81.4865) (end 165.1795 81.4865) (width 0.5) (layer "B.Cu") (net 2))
 (segment (start 177.689 121.428) (end 178.07 121.428) (width 0.5) (layer "B.Cu") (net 2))
 (segment (start 161.036 124.46) (end 161.036 82.55) (width 0.5) (layer "B.Cu") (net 2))
 (segment (start 179.197 125.095) (end 178.181 126.111) (width 0.5) (layer "B.Cu") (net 2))
 (segment (start 161.036 82.55) (end 162.0995 81.4865) (width 0.5) (layer "B.Cu") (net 2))
 (segment (start 162.687 126.111) (end 161.036 124.46) (width 0.5) (layer "B.Cu") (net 2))
 (segment (start 178.07 121.428) (end 179.197 122.555) (width 0.5) (layer "B.Cu") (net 2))
 (segment (start 177.689 116.348) (end 181.499 116.348) (width 1) (layer "F.Cu") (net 6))
 (segment (start 179.451 115.443) (end 179.451 109.347) (width 0.5) (layer "B.Cu") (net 6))
 (segment (start 177.562 107.458) (end 172.7995 107.458) (width 0.5) (layer "B.Cu") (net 6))
 (segment (start 179.451 109.347) (end 177.562 107.458) (width 0.5) (layer "B.Cu") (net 6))
 (segment (start 177.689 116.348) (end 178.546 116.348) (width 0.5) (layer "B.Cu") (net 6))
 (segment (start 178.546 116.348) (end 179.451 115.443) (width 0.5) (layer "B.Cu") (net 6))
 (segment (start 173.212 118.888) (end 176.276 115.824) (width 0.5) (layer "F.Cu") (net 4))
 (segment (start 176.276 114.3) (end 176.768 113.808) (width 0.5) (layer "F.Cu") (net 4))
 (segment (start 176.768 113.808) (end 177.689 113.808) (width 0.5) (layer "F.Cu") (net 4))
 (segment (start 172.085 118.888) (end 173.212 118.888) (width 0.5) (layer "F.Cu") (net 4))
 (segment (start 181.499 113.808) (end 177.689 113.808) (width 1) (layer "F.Cu") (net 4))
 (segment (start 176.276 115.824) (end 176.276 114.3) (width 0.5) (layer "F.Cu") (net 4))
 (segment (start 176.149 114.681) (end 176.149 121.539) (width 0.5) (layer "B.Cu") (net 4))
 (segment (start 176.149 121.539) (end 173.5455 124.1425) (width 0.5) (layer "B.Cu") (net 4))
 (segment (start 163.8935 124.1425) (end 173.5455 124.1425) (width 0.5) (layer "B.Cu") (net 4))
 (segment (start 177.689 113.808) (end 177.022 113.808) (width 0.5) (layer "B.Cu") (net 4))
 (segment (start 162.941 123.19) (end 162.941 92.837) (width 0.5) (layer "B.Cu") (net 4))
 (segment (start 177.022 113.808) (end 176.149 114.681) (width 0.5) (layer "B.Cu") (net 4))
 (segment (start 162.941 123.19) (end 163.8935 124.1425) (width 0.5) (layer "B.Cu") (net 4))
 (segment (start 162.941 92.837) (end 164.1315 91.6465) (width 0.5) (layer "B.Cu") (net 4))
 (segment (start 164.1315 91.6465) (end 165.1795 91.6465) (width 0.5) (layer "B.Cu") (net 4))
 (segment (start 162.433 96.139) (end 163.449 97.155) (width 0.5) (layer "F.Cu") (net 9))
 (segment (start 162.433 84.963) (end 162.433 96.139) (width 0.5) (layer "F.Cu") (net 9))
 (segment (start 163.3695 84.0265) (end 162.433 84.963) (width 0.5) (layer "F.Cu") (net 9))
 (segment (start 167.451 105.1865) (end 165.1795 107.458) (width 0.5) (layer "F.Cu") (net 9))
 (segment (start 163.449 97.155) (end 166.243 97.155) (width 0.5) (layer "F.Cu") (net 9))
 (segment (start 165.1795 84.0265) (end 163.3695 84.0265) (width 0.5) (layer "F.Cu") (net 9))
 (segment (start 166.243 97.155) (end 167.451 98.363) (width 0.5) (layer "F.Cu") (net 9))
 (segment (start 167.451 98.363) (end 167.451 105.1865) (width 0.5) (layer "F.Cu") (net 9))
 (segment (start 168.275 109.4425) (end 168.275 90.551) (width 0.5) (layer "F.Cu") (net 10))
 (segment (start 165.1795 112.538) (end 168.275 109.4425) (width 0.5) (layer "F.Cu") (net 10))
 (segment (start 168.275 90.551) (end 166.8305 89.1065) (width 0.5) (layer "F.Cu") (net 10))
 (segment (start 166.8305 89.1065) (end 165.1795 89.1065) (width 0.5) (layer "F.Cu") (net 10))
 (segment (start 166.751 98.933) (end 165.862 98.044) (width 0.5) (layer "F.Cu") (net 8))
 (segment (start 166.751 101.473) (end 166.751 98.933) (width 0.5) (layer "F.Cu") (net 8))
 (segment (start 163.3695 78.9465) (end 165.1795 78.9465) (width 0.5) (layer "F.Cu") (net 8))
 (segment (start 161.417 96.52) (end 161.417 80.899) (width 0.5) (layer "F.Cu") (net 8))
 (segment (start 165.1795 102.378) (end 165.846 102.378) (width 0.5) (layer "F.Cu") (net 8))
 (segment (start 161.417 80.899) (end 163.3695 78.9465) (width 0.5) (layer "F.Cu") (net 8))
 (segment (start 165.846 102.378) (end 166.751 101.473) (width 0.5) (layer "F.Cu") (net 8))
 (segment (start 165.862 98.044) (end 162.941 98.044) (width 0.5) (layer "F.Cu") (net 8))
 (segment (start 162.941 98.044) (end 161.417 96.52) (width 0.5) (layer "F.Cu") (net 8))
 (segment (start 172.7995 112.538) (end 172.7995 109.998) (width 0.5) (layer "F.Cu") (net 32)))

